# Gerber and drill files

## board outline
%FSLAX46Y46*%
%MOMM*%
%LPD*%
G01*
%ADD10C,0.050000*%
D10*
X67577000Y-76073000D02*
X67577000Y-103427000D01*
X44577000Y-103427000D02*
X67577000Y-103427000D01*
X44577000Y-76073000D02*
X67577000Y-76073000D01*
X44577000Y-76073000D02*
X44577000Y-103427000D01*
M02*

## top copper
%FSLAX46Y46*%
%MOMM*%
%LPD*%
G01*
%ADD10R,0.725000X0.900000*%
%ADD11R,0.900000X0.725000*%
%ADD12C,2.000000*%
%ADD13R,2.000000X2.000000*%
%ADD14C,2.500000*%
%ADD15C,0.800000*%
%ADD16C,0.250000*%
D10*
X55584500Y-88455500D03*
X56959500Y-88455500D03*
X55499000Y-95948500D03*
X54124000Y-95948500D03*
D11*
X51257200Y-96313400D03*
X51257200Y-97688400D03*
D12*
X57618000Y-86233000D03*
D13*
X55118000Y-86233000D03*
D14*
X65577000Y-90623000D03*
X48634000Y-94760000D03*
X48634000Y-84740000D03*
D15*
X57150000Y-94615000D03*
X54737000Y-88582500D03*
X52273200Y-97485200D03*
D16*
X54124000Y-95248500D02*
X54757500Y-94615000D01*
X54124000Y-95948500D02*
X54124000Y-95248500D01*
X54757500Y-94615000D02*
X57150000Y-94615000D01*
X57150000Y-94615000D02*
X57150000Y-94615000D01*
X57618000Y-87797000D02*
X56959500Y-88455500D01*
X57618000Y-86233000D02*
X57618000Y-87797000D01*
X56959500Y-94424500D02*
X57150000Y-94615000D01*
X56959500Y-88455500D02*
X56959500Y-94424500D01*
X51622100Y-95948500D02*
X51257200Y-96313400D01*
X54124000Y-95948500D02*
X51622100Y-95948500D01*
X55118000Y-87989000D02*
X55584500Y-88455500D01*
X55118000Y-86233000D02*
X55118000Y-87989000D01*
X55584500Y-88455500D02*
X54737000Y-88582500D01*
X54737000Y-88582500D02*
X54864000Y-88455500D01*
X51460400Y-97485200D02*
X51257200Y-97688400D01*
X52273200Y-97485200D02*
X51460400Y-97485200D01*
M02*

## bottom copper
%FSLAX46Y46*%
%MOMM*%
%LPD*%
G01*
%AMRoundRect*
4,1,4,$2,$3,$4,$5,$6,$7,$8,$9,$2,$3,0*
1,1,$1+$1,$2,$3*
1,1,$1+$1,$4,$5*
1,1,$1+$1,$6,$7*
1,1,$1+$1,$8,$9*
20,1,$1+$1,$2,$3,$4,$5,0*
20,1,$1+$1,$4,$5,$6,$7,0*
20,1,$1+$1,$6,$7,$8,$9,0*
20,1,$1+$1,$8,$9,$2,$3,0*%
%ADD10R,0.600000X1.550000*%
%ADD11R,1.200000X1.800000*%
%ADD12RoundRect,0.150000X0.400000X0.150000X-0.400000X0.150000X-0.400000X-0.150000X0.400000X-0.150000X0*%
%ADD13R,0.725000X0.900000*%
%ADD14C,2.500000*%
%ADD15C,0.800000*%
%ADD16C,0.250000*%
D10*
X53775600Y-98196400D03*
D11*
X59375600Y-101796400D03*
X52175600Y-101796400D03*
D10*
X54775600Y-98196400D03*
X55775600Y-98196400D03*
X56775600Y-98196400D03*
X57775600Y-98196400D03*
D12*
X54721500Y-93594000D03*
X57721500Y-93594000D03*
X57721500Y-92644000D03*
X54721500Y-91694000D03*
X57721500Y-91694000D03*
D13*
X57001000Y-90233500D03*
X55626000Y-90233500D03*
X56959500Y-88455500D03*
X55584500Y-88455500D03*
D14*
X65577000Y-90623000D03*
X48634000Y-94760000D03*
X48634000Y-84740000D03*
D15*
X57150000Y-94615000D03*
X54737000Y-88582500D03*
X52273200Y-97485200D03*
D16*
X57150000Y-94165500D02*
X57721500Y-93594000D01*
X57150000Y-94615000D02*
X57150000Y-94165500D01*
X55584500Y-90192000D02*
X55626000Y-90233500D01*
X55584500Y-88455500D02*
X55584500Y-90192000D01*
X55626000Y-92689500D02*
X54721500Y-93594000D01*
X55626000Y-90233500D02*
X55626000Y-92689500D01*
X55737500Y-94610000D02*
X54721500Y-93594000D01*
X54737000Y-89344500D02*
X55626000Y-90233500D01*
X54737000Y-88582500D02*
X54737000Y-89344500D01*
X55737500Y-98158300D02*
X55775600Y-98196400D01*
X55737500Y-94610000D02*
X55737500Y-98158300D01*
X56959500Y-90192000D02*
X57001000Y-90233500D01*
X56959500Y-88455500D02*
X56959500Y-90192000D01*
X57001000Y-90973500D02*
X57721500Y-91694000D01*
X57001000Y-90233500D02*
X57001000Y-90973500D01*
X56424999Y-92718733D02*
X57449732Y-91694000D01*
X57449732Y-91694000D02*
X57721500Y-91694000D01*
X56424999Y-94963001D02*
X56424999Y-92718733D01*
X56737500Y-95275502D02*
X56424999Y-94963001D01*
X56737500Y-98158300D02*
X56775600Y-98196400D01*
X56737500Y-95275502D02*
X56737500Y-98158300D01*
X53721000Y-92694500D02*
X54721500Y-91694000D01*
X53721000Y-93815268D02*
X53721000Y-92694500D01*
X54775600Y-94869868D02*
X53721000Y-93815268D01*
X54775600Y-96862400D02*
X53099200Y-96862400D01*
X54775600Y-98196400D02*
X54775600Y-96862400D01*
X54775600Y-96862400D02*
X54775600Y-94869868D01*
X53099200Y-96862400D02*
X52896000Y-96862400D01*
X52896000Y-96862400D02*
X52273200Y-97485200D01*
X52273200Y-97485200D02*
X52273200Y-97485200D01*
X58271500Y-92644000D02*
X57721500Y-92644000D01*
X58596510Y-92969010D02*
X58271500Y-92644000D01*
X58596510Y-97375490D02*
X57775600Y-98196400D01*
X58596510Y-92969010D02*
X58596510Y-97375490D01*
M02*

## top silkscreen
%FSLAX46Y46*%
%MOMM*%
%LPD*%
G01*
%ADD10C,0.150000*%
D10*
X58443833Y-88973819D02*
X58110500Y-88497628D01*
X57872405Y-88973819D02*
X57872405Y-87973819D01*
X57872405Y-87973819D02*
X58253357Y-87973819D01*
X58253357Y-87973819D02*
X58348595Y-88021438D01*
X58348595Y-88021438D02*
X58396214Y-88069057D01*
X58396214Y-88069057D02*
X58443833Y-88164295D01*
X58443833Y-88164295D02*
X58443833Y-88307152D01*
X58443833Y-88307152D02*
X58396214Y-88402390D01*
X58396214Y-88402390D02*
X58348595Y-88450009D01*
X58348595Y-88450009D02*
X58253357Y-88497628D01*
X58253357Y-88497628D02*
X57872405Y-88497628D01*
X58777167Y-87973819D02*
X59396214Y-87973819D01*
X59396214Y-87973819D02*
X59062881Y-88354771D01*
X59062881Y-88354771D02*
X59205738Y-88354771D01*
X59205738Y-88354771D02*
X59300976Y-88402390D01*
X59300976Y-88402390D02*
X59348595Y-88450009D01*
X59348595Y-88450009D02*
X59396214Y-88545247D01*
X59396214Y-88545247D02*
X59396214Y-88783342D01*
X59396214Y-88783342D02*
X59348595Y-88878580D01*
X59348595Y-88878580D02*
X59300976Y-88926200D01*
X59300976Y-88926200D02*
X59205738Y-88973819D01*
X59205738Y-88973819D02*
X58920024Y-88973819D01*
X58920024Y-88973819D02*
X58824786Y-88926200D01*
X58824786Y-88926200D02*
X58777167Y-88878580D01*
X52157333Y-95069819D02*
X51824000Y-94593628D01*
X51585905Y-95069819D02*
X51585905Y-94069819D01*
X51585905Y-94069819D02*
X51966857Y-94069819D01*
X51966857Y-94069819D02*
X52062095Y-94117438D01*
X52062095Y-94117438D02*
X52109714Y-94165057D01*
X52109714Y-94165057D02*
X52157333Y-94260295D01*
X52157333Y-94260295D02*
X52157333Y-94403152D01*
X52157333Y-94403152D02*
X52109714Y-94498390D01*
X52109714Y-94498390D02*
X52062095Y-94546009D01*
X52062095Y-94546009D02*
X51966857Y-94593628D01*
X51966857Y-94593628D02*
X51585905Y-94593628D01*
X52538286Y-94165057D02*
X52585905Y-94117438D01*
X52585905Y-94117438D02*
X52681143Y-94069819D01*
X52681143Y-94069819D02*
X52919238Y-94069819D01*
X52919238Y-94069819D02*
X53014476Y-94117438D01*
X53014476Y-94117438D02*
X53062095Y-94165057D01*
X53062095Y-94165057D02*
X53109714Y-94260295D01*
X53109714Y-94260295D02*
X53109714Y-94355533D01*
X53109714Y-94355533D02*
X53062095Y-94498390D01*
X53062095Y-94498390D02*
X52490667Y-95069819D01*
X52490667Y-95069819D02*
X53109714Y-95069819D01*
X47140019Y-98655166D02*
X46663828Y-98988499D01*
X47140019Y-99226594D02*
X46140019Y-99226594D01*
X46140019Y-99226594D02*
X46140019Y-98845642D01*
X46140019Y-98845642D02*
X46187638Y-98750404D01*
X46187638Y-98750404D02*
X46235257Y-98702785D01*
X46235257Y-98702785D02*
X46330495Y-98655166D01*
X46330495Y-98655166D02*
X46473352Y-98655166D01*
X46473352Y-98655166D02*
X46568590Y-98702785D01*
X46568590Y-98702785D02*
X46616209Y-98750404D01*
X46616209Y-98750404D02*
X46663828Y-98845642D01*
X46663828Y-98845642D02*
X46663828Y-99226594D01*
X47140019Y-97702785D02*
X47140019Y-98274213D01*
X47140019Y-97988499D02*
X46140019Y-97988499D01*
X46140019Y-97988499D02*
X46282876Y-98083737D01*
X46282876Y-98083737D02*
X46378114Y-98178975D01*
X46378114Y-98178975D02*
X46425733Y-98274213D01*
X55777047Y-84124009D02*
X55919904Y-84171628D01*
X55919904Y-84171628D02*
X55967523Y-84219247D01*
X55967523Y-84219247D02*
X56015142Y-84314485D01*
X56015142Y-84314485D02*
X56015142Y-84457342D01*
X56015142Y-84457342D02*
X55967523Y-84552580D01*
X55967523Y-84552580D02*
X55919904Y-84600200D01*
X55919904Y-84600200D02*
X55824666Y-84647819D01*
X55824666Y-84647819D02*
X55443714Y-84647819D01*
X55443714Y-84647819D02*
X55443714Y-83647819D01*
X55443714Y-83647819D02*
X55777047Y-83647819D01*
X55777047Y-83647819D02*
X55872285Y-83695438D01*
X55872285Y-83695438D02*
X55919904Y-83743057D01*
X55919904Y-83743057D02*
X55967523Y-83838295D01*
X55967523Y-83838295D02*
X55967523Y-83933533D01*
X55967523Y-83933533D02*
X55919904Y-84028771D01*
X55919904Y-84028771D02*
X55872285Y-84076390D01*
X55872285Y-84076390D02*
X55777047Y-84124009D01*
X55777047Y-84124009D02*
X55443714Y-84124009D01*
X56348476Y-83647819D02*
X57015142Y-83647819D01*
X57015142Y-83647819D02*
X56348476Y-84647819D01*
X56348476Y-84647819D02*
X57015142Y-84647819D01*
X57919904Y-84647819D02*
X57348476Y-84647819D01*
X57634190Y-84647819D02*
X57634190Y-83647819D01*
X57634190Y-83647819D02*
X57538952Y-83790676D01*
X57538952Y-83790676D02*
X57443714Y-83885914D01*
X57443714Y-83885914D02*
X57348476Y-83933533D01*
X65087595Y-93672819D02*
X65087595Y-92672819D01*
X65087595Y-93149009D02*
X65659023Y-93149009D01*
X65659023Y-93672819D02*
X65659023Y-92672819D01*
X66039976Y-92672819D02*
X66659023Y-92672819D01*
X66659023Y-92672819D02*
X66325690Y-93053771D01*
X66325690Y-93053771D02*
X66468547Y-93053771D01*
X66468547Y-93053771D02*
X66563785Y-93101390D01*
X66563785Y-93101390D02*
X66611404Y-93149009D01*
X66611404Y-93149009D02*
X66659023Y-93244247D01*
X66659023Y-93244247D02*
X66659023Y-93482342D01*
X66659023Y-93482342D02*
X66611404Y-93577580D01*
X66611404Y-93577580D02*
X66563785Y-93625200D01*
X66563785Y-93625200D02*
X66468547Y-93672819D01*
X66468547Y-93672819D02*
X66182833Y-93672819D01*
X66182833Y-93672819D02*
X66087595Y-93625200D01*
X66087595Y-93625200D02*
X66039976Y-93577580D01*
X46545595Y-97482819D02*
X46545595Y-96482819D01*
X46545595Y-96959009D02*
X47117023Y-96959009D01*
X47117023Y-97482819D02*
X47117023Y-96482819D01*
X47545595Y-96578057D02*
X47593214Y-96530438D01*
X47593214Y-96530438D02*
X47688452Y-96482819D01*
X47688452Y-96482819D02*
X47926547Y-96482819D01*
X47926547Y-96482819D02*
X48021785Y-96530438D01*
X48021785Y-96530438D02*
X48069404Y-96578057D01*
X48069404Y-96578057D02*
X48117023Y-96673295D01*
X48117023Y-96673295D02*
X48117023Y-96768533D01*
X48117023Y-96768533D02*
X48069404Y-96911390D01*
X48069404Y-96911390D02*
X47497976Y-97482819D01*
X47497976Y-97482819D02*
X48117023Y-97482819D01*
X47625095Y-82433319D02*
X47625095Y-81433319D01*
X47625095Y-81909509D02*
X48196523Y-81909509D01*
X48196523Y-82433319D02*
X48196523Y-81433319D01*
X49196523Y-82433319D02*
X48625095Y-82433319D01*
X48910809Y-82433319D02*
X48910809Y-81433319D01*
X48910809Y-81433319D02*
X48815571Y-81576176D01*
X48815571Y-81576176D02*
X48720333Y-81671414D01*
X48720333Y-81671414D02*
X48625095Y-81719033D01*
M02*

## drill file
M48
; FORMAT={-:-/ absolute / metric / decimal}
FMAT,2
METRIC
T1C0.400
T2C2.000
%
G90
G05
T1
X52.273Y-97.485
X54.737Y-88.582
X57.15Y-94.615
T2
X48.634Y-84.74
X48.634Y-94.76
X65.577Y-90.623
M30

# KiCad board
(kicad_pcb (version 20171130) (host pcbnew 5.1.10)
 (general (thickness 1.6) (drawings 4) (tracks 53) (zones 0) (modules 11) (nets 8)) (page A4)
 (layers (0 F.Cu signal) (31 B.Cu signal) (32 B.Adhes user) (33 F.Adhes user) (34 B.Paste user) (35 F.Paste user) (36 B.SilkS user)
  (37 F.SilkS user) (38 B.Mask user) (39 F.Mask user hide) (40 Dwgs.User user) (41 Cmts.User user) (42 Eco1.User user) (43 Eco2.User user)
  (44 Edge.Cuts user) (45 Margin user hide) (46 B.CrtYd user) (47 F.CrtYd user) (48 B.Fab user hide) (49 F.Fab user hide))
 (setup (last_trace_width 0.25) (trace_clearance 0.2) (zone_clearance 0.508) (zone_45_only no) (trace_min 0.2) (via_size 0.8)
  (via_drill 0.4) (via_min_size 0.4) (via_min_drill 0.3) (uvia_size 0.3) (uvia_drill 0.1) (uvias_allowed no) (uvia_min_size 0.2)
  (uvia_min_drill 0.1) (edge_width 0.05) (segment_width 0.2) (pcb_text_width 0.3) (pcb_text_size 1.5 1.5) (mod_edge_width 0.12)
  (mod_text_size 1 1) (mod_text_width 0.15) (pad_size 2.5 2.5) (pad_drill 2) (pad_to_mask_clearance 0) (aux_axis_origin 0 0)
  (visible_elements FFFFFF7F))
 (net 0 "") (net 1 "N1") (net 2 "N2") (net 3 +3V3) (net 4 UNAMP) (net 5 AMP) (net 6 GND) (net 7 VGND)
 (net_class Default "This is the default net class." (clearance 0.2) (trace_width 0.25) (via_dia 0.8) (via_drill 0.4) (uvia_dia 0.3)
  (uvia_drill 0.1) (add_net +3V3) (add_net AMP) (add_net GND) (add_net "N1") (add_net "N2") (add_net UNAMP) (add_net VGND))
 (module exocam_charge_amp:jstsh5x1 (layer B.Cu) (at 54.9656 95.6564 180)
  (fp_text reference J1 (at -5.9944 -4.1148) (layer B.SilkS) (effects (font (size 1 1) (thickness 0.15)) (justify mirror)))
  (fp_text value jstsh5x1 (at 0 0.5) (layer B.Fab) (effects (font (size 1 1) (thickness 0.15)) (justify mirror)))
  (pad 5 smd rect (at 1.19 -2.54 180) (size 0.6 1.55) (layers B.Cu B.Paste B.Mask) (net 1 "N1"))
  (pad 6 smd rect (at -4.41 -6.14 180) (size 1.2 1.8) (layers B.Cu B.Paste B.Mask) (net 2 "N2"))
  (pad 6 smd rect (at 2.79 -6.14 180) (size 1.2 1.8) (layers B.Cu B.Paste B.Mask) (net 2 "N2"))
  (pad 4 smd rect (at 0.19 -2.54 180) (size 0.6 1.55) (layers B.Cu B.Paste B.Mask) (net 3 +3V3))
  (pad 3 smd rect (at -0.81 -2.54 180) (size 0.6 1.55) (layers B.Cu B.Paste B.Mask) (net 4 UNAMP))
  (pad 2 smd rect (at -1.81 -2.54 180) (size 0.6 1.55) (layers B.Cu B.Paste B.Mask) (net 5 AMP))
  (pad 1 smd rect (at -2.81 -2.54 180) (size 0.6 1.55) (layers B.Cu B.Paste B.Mask) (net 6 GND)))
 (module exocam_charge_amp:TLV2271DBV (layer B.Cu) (at 56.4515 89.154 180)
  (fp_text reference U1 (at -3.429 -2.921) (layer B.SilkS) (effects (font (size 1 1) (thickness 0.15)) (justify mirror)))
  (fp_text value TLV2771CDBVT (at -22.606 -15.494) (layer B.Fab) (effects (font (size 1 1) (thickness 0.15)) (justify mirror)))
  (pad 4 smd roundrect (at 1.73 -4.44 180) (size 1.1 0.6) (layers B.Cu B.Paste B.Mask) (roundrect_rratio 0.25) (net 4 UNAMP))
  (pad 3 smd roundrect (at -1.27 -4.44 180) (size 1.1 0.6) (layers B.Cu B.Paste B.Mask) (roundrect_rratio 0.25) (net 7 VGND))
  (pad 2 smd roundrect (at -1.27 -3.49 180) (size 1.1 0.6) (layers B.Cu B.Paste B.Mask) (roundrect_rratio 0.25) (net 6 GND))
  (pad 5 smd roundrect (at 1.73 -2.54 180) (size 1.1 0.6) (layers B.Cu B.Paste B.Mask) (roundrect_rratio 0.25) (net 3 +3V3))
  (pad 1 smd roundrect (at -1.27 -2.54 180) (size 1.1 0.6) (layers B.Cu B.Paste B.Mask) (roundrect_rratio 0.25) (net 5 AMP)))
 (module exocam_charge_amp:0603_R (layer B.Cu) (at 56.896 92.7735)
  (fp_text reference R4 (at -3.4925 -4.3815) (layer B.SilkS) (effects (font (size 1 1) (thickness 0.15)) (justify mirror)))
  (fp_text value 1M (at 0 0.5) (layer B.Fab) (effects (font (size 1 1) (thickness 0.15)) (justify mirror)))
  (pad 2 smd rect (at 0.105 -2.54) (size 0.725 0.9) (layers B.Cu B.Paste B.Mask) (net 5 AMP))
  (pad 1 smd rect (at -1.27 -2.54) (size 0.725 0.9) (layers B.Cu B.Paste B.Mask) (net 4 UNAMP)))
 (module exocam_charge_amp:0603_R (layer F.Cu) (at 55.6895 90.9955 180)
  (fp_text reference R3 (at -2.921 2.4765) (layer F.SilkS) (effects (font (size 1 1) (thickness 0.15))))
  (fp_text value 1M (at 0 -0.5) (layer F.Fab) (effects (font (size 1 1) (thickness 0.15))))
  (pad 2 smd rect (at 0.105 2.54 180) (size 0.725 0.9) (layers F.Cu F.Paste F.Mask) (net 4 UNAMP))
  (pad 1 smd rect (at -1.27 2.54 180) (size 0.725 0.9) (layers F.Cu F.Paste F.Mask) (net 7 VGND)))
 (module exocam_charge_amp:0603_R (layer F.Cu) (at 55.394 93.4085)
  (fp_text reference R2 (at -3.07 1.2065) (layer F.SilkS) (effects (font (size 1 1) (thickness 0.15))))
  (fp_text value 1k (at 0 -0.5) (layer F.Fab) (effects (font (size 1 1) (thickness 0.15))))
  (pad 2 smd rect (at 0.105 2.54) (size 0.725 0.9) (layers F.Cu F.Paste F.Mask) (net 6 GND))
  (pad 1 smd rect (at -1.27 2.54) (size 0.725 0.9) (layers F.Cu F.Paste F.Mask) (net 7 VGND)))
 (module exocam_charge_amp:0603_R (layer F.Cu) (at 48.7172 96.4184 90)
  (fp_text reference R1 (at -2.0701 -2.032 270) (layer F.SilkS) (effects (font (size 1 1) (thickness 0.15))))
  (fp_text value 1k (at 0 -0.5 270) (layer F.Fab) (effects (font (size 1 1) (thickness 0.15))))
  (pad 2 smd rect (at 0.105 2.54 90) (size 0.725 0.9) (layers F.Cu F.Paste F.Mask) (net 7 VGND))
  (pad 1 smd rect (at -1.27 2.54 90) (size 0.725 0.9) (layers F.Cu F.Paste F.Mask) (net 3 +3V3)))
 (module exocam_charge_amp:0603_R (layer B.Cu) (at 56.8545 90.9955)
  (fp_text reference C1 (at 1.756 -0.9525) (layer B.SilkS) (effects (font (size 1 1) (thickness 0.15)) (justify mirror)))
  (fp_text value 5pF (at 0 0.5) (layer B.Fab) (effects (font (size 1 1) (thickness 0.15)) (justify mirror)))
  (pad 2 smd rect (at 0.105 -2.54) (size 0.725 0.9) (layers B.Cu B.Paste B.Mask) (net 5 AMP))
  (pad 1 smd rect (at -1.27 -2.54) (size 0.725 0.9) (layers B.Cu B.Paste B.Mask) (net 4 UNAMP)))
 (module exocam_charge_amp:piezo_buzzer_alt (layer F.Cu) (at 56.658 83.693)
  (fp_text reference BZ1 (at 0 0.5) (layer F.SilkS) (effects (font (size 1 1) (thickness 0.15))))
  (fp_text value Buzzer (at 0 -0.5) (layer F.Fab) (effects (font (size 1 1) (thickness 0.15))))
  (pad 2 smd circle (at 0.96 2.54) (size 2 2) (layers F.Cu F.Paste F.Mask) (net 7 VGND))
  (pad 1 smd rect (at -1.54 2.54) (size 2 2) (layers F.Cu F.Paste F.Mask) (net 4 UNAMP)))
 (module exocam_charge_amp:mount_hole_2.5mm (layer F.Cu) (at 60.1815 91.44)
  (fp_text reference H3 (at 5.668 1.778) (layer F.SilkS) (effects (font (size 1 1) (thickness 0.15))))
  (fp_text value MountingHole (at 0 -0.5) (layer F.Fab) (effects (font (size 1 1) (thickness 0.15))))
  (pad 1 thru_hole circle (at 5.3955 -0.817) (size 2.5 2.5) (drill 2) (layers *.Cu *.Mask)))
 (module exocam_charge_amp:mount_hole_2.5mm (layer F.Cu) (at 48.7045 94.9325)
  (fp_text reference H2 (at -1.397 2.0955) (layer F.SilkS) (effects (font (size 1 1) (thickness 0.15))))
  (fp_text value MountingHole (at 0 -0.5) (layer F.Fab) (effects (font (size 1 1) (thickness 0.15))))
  (pad 1 thru_hole circle (at -0.0705 -0.1725) (size 2.5 2.5) (drill 2) (layers *.Cu *.Mask)))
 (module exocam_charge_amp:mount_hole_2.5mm (layer F.Cu) (at 48.641 75.565)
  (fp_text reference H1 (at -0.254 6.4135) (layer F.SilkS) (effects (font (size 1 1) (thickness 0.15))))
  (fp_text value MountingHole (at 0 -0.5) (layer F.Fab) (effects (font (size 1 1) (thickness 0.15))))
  (pad 1 thru_hole circle (at -0.007 9.175) (size 2.5 2.5) (drill 2) (layers *.Cu *.Mask)))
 (gr_line (start 67.577 76.073) (end 67.577 103.427) (layer Edge.Cuts) (width 0.05))
 (gr_line (start 44.577 103.427) (end 67.577 103.427) (layer Edge.Cuts) (width 0.05))
 (gr_line (start 44.577 76.073) (end 67.577 76.073) (layer Edge.Cuts) (width 0.05))
 (gr_line (start 44.577 76.073) (end 44.577 103.427) (layer Edge.Cuts) (width 0.05))
 (segment (start 54.124 95.2485) (end 54.7575 94.615) (width 0.25) (layer F.Cu) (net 7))
 (segment (start 54.124 95.9485) (end 54.124 95.2485) (width 0.25) (layer F.Cu) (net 7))
 (segment (start 54.7575 94.615) (end 57.15 94.615) (width 0.25) (layer F.Cu) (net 7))
 (segment (start 57.15 94.615) (end 57.15 94.615) (width 0.25) (layer F.Cu) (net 7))
 (via (at 57.15 94.615) (size 0.8) (drill 0.4) (layers F.Cu B.Cu) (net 7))
 (segment (start 57.15 94.1655) (end 57.7215 93.594) (width 0.25) (layer B.Cu) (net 7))
 (segment (start 57.15 94.615) (end 57.15 94.1655) (width 0.25) (layer B.Cu) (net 7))
 (segment (start 57.618 87.797) (end 56.9595 88.4555) (width 0.25) (layer F.Cu) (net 7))
 (segment (start 57.618 86.233) (end 57.618 87.797) (width 0.25) (layer F.Cu) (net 7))
 (segment (start 56.9595 94.4245) (end 57.15 94.615) (width 0.25) (layer F.Cu) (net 7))
 (segment (start 56.9595 88.4555) (end 56.9595 94.4245) (width 0.25) (layer F.Cu) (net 7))
 (segment (start 51.6221 95.9485) (end 51.2572 96.3134) (width 0.25) (layer F.Cu) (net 7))
 (segment (start 54.124 95.9485) (end 51.6221 95.9485) (width 0.25) (layer F.Cu) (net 7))
 (segment (start 55.5845 90.192) (end 55.626 90.2335) (width 0.25) (layer B.Cu) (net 4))
 (segment (start 55.5845 88.4555) (end 55.5845 90.192) (width 0.25) (layer B.Cu) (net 4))
 (segment (start 55.626 92.6895) (end 54.7215 93.594) (width 0.25) (layer B.Cu) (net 4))
 (segment (start 55.626 90.2335) (end 55.626 92.6895) (width 0.25) (layer B.Cu) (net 4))
 (segment (start 55.7375 94.61) (end 54.7215 93.594) (width 0.25) (layer B.Cu) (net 4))
 (segment (start 55.118 87.989) (end 55.5845 88.4555) (width 0.25) (layer F.Cu) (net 4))
 (segment (start 55.118 86.233) (end 55.118 87.989) (width 0.25) (layer F.Cu) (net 4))
 (segment (start 55.5845 88.4555) (end 54.737 88.5825) (width 0.25) (layer F.Cu) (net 4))
 (segment (start 54.737 88.5825) (end 54.864 88.4555) (width 0.25) (layer F.Cu) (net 4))
 (via (at 54.737 88.5825) (size 0.8) (drill 0.4) (layers F.Cu B.Cu) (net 4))
 (segment (start 54.737 89.3445) (end 55.626 90.2335) (width 0.25) (layer B.Cu) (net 4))
 (segment (start 54.737 88.5825) (end 54.737 89.3445) (width 0.25) (layer B.Cu) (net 4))
 (segment (start 55.7375 98.1583) (end 55.7756 98.1964) (width 0.25) (layer B.Cu) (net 4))
 (segment (start 55.7375 94.61) (end 55.7375 98.1583) (width 0.25) (layer B.Cu) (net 4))
 (segment (start 56.9595 90.192) (end 57.001 90.2335) (width 0.25) (layer B.Cu) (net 5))
 (segment (start 56.9595 88.4555) (end 56.9595 90.192) (width 0.25) (layer B.Cu) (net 5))
 (segment (start 57.001 90.9735) (end 57.7215 91.694) (width 0.25) (layer B.Cu) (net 5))
 (segment (start 57.001 90.2335) (end 57.001 90.9735) (width 0.25) (layer B.Cu) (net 5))
 (segment (start 56.424999 92.718733) (end 57.449732 91.694) (width 0.25) (layer B.Cu) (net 5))
 (segment (start 57.449732 91.694) (end 57.7215 91.694) (width 0.25) (layer B.Cu) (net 5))
 (segment (start 56.424999 94.963001) (end 56.424999 92.718733) (width 0.25) (layer B.Cu) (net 5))
 (segment (start 56.7375 95.275502) (end 56.424999 94.963001) (width 0.25) (layer B.Cu) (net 5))
 (segment (start 56.7375 98.1583) (end 56.7756 98.1964) (width 0.25) (layer B.Cu) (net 5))
 (segment (start 56.7375 95.275502) (end 56.7375 98.1583) (width 0.25) (layer B.Cu) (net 5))
 (segment (start 53.721 92.6945) (end 54.7215 91.694) (width 0.25) (layer B.Cu) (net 3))
 (segment (start 53.721 93.815268) (end 53.721 92.6945) (width 0.25) (layer B.Cu) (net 3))
 (segment (start 54.7756 94.869868) (end 53.721 93.815268) (width 0.25) (layer B.Cu) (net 3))
 (segment (start 54.7756 96.8624) (end 53.0992 96.8624) (width 0.25) (layer B.Cu) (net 3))
 (segment (start 54.7756 98.1964) (end 54.7756 96.8624) (width 0.25) (layer B.Cu) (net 3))
 (segment (start 54.7756 96.8624) (end 54.7756 94.869868) (width 0.25) (layer B.Cu) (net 3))
 (segment (start 53.0992 96.8624) (end 52.896 96.8624) (width 0.25) (layer B.Cu) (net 3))
 (segment (start 52.896 96.8624) (end 52.2732 97.4852) (width 0.25) (layer B.Cu) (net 3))
 (segment (start 52.2732 97.4852) (end 52.2732 97.4852) (width 0.25) (layer B.Cu) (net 3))
 (via (at 52.2732 97.4852) (size 0.8) (drill 0.4) (layers F.Cu B.Cu) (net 3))
 (segment (start 51.4604 97.4852) (end 51.2572 97.6884) (width 0.25) (layer F.Cu) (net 3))
 (segment (start 52.2732 97.4852) (end 51.4604 97.4852) (width 0.25) (layer F.Cu) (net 3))
 (segment (start 58.2715 92.644) (end 57.7215 92.644) (width 0.25) (layer B.Cu) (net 6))
 (segment (start 58.59651 92.96901) (end 58.2715 92.644) (width 0.25) (layer B.Cu) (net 6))
 (segment (start 58.59651 97.37549) (end 57.7756 98.1964) (width 0.25) (layer B.Cu) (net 6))
 (segment (start 58.59651 92.96901) (end 58.59651 97.37549) (width 0.25) (layer B.Cu) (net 6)))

